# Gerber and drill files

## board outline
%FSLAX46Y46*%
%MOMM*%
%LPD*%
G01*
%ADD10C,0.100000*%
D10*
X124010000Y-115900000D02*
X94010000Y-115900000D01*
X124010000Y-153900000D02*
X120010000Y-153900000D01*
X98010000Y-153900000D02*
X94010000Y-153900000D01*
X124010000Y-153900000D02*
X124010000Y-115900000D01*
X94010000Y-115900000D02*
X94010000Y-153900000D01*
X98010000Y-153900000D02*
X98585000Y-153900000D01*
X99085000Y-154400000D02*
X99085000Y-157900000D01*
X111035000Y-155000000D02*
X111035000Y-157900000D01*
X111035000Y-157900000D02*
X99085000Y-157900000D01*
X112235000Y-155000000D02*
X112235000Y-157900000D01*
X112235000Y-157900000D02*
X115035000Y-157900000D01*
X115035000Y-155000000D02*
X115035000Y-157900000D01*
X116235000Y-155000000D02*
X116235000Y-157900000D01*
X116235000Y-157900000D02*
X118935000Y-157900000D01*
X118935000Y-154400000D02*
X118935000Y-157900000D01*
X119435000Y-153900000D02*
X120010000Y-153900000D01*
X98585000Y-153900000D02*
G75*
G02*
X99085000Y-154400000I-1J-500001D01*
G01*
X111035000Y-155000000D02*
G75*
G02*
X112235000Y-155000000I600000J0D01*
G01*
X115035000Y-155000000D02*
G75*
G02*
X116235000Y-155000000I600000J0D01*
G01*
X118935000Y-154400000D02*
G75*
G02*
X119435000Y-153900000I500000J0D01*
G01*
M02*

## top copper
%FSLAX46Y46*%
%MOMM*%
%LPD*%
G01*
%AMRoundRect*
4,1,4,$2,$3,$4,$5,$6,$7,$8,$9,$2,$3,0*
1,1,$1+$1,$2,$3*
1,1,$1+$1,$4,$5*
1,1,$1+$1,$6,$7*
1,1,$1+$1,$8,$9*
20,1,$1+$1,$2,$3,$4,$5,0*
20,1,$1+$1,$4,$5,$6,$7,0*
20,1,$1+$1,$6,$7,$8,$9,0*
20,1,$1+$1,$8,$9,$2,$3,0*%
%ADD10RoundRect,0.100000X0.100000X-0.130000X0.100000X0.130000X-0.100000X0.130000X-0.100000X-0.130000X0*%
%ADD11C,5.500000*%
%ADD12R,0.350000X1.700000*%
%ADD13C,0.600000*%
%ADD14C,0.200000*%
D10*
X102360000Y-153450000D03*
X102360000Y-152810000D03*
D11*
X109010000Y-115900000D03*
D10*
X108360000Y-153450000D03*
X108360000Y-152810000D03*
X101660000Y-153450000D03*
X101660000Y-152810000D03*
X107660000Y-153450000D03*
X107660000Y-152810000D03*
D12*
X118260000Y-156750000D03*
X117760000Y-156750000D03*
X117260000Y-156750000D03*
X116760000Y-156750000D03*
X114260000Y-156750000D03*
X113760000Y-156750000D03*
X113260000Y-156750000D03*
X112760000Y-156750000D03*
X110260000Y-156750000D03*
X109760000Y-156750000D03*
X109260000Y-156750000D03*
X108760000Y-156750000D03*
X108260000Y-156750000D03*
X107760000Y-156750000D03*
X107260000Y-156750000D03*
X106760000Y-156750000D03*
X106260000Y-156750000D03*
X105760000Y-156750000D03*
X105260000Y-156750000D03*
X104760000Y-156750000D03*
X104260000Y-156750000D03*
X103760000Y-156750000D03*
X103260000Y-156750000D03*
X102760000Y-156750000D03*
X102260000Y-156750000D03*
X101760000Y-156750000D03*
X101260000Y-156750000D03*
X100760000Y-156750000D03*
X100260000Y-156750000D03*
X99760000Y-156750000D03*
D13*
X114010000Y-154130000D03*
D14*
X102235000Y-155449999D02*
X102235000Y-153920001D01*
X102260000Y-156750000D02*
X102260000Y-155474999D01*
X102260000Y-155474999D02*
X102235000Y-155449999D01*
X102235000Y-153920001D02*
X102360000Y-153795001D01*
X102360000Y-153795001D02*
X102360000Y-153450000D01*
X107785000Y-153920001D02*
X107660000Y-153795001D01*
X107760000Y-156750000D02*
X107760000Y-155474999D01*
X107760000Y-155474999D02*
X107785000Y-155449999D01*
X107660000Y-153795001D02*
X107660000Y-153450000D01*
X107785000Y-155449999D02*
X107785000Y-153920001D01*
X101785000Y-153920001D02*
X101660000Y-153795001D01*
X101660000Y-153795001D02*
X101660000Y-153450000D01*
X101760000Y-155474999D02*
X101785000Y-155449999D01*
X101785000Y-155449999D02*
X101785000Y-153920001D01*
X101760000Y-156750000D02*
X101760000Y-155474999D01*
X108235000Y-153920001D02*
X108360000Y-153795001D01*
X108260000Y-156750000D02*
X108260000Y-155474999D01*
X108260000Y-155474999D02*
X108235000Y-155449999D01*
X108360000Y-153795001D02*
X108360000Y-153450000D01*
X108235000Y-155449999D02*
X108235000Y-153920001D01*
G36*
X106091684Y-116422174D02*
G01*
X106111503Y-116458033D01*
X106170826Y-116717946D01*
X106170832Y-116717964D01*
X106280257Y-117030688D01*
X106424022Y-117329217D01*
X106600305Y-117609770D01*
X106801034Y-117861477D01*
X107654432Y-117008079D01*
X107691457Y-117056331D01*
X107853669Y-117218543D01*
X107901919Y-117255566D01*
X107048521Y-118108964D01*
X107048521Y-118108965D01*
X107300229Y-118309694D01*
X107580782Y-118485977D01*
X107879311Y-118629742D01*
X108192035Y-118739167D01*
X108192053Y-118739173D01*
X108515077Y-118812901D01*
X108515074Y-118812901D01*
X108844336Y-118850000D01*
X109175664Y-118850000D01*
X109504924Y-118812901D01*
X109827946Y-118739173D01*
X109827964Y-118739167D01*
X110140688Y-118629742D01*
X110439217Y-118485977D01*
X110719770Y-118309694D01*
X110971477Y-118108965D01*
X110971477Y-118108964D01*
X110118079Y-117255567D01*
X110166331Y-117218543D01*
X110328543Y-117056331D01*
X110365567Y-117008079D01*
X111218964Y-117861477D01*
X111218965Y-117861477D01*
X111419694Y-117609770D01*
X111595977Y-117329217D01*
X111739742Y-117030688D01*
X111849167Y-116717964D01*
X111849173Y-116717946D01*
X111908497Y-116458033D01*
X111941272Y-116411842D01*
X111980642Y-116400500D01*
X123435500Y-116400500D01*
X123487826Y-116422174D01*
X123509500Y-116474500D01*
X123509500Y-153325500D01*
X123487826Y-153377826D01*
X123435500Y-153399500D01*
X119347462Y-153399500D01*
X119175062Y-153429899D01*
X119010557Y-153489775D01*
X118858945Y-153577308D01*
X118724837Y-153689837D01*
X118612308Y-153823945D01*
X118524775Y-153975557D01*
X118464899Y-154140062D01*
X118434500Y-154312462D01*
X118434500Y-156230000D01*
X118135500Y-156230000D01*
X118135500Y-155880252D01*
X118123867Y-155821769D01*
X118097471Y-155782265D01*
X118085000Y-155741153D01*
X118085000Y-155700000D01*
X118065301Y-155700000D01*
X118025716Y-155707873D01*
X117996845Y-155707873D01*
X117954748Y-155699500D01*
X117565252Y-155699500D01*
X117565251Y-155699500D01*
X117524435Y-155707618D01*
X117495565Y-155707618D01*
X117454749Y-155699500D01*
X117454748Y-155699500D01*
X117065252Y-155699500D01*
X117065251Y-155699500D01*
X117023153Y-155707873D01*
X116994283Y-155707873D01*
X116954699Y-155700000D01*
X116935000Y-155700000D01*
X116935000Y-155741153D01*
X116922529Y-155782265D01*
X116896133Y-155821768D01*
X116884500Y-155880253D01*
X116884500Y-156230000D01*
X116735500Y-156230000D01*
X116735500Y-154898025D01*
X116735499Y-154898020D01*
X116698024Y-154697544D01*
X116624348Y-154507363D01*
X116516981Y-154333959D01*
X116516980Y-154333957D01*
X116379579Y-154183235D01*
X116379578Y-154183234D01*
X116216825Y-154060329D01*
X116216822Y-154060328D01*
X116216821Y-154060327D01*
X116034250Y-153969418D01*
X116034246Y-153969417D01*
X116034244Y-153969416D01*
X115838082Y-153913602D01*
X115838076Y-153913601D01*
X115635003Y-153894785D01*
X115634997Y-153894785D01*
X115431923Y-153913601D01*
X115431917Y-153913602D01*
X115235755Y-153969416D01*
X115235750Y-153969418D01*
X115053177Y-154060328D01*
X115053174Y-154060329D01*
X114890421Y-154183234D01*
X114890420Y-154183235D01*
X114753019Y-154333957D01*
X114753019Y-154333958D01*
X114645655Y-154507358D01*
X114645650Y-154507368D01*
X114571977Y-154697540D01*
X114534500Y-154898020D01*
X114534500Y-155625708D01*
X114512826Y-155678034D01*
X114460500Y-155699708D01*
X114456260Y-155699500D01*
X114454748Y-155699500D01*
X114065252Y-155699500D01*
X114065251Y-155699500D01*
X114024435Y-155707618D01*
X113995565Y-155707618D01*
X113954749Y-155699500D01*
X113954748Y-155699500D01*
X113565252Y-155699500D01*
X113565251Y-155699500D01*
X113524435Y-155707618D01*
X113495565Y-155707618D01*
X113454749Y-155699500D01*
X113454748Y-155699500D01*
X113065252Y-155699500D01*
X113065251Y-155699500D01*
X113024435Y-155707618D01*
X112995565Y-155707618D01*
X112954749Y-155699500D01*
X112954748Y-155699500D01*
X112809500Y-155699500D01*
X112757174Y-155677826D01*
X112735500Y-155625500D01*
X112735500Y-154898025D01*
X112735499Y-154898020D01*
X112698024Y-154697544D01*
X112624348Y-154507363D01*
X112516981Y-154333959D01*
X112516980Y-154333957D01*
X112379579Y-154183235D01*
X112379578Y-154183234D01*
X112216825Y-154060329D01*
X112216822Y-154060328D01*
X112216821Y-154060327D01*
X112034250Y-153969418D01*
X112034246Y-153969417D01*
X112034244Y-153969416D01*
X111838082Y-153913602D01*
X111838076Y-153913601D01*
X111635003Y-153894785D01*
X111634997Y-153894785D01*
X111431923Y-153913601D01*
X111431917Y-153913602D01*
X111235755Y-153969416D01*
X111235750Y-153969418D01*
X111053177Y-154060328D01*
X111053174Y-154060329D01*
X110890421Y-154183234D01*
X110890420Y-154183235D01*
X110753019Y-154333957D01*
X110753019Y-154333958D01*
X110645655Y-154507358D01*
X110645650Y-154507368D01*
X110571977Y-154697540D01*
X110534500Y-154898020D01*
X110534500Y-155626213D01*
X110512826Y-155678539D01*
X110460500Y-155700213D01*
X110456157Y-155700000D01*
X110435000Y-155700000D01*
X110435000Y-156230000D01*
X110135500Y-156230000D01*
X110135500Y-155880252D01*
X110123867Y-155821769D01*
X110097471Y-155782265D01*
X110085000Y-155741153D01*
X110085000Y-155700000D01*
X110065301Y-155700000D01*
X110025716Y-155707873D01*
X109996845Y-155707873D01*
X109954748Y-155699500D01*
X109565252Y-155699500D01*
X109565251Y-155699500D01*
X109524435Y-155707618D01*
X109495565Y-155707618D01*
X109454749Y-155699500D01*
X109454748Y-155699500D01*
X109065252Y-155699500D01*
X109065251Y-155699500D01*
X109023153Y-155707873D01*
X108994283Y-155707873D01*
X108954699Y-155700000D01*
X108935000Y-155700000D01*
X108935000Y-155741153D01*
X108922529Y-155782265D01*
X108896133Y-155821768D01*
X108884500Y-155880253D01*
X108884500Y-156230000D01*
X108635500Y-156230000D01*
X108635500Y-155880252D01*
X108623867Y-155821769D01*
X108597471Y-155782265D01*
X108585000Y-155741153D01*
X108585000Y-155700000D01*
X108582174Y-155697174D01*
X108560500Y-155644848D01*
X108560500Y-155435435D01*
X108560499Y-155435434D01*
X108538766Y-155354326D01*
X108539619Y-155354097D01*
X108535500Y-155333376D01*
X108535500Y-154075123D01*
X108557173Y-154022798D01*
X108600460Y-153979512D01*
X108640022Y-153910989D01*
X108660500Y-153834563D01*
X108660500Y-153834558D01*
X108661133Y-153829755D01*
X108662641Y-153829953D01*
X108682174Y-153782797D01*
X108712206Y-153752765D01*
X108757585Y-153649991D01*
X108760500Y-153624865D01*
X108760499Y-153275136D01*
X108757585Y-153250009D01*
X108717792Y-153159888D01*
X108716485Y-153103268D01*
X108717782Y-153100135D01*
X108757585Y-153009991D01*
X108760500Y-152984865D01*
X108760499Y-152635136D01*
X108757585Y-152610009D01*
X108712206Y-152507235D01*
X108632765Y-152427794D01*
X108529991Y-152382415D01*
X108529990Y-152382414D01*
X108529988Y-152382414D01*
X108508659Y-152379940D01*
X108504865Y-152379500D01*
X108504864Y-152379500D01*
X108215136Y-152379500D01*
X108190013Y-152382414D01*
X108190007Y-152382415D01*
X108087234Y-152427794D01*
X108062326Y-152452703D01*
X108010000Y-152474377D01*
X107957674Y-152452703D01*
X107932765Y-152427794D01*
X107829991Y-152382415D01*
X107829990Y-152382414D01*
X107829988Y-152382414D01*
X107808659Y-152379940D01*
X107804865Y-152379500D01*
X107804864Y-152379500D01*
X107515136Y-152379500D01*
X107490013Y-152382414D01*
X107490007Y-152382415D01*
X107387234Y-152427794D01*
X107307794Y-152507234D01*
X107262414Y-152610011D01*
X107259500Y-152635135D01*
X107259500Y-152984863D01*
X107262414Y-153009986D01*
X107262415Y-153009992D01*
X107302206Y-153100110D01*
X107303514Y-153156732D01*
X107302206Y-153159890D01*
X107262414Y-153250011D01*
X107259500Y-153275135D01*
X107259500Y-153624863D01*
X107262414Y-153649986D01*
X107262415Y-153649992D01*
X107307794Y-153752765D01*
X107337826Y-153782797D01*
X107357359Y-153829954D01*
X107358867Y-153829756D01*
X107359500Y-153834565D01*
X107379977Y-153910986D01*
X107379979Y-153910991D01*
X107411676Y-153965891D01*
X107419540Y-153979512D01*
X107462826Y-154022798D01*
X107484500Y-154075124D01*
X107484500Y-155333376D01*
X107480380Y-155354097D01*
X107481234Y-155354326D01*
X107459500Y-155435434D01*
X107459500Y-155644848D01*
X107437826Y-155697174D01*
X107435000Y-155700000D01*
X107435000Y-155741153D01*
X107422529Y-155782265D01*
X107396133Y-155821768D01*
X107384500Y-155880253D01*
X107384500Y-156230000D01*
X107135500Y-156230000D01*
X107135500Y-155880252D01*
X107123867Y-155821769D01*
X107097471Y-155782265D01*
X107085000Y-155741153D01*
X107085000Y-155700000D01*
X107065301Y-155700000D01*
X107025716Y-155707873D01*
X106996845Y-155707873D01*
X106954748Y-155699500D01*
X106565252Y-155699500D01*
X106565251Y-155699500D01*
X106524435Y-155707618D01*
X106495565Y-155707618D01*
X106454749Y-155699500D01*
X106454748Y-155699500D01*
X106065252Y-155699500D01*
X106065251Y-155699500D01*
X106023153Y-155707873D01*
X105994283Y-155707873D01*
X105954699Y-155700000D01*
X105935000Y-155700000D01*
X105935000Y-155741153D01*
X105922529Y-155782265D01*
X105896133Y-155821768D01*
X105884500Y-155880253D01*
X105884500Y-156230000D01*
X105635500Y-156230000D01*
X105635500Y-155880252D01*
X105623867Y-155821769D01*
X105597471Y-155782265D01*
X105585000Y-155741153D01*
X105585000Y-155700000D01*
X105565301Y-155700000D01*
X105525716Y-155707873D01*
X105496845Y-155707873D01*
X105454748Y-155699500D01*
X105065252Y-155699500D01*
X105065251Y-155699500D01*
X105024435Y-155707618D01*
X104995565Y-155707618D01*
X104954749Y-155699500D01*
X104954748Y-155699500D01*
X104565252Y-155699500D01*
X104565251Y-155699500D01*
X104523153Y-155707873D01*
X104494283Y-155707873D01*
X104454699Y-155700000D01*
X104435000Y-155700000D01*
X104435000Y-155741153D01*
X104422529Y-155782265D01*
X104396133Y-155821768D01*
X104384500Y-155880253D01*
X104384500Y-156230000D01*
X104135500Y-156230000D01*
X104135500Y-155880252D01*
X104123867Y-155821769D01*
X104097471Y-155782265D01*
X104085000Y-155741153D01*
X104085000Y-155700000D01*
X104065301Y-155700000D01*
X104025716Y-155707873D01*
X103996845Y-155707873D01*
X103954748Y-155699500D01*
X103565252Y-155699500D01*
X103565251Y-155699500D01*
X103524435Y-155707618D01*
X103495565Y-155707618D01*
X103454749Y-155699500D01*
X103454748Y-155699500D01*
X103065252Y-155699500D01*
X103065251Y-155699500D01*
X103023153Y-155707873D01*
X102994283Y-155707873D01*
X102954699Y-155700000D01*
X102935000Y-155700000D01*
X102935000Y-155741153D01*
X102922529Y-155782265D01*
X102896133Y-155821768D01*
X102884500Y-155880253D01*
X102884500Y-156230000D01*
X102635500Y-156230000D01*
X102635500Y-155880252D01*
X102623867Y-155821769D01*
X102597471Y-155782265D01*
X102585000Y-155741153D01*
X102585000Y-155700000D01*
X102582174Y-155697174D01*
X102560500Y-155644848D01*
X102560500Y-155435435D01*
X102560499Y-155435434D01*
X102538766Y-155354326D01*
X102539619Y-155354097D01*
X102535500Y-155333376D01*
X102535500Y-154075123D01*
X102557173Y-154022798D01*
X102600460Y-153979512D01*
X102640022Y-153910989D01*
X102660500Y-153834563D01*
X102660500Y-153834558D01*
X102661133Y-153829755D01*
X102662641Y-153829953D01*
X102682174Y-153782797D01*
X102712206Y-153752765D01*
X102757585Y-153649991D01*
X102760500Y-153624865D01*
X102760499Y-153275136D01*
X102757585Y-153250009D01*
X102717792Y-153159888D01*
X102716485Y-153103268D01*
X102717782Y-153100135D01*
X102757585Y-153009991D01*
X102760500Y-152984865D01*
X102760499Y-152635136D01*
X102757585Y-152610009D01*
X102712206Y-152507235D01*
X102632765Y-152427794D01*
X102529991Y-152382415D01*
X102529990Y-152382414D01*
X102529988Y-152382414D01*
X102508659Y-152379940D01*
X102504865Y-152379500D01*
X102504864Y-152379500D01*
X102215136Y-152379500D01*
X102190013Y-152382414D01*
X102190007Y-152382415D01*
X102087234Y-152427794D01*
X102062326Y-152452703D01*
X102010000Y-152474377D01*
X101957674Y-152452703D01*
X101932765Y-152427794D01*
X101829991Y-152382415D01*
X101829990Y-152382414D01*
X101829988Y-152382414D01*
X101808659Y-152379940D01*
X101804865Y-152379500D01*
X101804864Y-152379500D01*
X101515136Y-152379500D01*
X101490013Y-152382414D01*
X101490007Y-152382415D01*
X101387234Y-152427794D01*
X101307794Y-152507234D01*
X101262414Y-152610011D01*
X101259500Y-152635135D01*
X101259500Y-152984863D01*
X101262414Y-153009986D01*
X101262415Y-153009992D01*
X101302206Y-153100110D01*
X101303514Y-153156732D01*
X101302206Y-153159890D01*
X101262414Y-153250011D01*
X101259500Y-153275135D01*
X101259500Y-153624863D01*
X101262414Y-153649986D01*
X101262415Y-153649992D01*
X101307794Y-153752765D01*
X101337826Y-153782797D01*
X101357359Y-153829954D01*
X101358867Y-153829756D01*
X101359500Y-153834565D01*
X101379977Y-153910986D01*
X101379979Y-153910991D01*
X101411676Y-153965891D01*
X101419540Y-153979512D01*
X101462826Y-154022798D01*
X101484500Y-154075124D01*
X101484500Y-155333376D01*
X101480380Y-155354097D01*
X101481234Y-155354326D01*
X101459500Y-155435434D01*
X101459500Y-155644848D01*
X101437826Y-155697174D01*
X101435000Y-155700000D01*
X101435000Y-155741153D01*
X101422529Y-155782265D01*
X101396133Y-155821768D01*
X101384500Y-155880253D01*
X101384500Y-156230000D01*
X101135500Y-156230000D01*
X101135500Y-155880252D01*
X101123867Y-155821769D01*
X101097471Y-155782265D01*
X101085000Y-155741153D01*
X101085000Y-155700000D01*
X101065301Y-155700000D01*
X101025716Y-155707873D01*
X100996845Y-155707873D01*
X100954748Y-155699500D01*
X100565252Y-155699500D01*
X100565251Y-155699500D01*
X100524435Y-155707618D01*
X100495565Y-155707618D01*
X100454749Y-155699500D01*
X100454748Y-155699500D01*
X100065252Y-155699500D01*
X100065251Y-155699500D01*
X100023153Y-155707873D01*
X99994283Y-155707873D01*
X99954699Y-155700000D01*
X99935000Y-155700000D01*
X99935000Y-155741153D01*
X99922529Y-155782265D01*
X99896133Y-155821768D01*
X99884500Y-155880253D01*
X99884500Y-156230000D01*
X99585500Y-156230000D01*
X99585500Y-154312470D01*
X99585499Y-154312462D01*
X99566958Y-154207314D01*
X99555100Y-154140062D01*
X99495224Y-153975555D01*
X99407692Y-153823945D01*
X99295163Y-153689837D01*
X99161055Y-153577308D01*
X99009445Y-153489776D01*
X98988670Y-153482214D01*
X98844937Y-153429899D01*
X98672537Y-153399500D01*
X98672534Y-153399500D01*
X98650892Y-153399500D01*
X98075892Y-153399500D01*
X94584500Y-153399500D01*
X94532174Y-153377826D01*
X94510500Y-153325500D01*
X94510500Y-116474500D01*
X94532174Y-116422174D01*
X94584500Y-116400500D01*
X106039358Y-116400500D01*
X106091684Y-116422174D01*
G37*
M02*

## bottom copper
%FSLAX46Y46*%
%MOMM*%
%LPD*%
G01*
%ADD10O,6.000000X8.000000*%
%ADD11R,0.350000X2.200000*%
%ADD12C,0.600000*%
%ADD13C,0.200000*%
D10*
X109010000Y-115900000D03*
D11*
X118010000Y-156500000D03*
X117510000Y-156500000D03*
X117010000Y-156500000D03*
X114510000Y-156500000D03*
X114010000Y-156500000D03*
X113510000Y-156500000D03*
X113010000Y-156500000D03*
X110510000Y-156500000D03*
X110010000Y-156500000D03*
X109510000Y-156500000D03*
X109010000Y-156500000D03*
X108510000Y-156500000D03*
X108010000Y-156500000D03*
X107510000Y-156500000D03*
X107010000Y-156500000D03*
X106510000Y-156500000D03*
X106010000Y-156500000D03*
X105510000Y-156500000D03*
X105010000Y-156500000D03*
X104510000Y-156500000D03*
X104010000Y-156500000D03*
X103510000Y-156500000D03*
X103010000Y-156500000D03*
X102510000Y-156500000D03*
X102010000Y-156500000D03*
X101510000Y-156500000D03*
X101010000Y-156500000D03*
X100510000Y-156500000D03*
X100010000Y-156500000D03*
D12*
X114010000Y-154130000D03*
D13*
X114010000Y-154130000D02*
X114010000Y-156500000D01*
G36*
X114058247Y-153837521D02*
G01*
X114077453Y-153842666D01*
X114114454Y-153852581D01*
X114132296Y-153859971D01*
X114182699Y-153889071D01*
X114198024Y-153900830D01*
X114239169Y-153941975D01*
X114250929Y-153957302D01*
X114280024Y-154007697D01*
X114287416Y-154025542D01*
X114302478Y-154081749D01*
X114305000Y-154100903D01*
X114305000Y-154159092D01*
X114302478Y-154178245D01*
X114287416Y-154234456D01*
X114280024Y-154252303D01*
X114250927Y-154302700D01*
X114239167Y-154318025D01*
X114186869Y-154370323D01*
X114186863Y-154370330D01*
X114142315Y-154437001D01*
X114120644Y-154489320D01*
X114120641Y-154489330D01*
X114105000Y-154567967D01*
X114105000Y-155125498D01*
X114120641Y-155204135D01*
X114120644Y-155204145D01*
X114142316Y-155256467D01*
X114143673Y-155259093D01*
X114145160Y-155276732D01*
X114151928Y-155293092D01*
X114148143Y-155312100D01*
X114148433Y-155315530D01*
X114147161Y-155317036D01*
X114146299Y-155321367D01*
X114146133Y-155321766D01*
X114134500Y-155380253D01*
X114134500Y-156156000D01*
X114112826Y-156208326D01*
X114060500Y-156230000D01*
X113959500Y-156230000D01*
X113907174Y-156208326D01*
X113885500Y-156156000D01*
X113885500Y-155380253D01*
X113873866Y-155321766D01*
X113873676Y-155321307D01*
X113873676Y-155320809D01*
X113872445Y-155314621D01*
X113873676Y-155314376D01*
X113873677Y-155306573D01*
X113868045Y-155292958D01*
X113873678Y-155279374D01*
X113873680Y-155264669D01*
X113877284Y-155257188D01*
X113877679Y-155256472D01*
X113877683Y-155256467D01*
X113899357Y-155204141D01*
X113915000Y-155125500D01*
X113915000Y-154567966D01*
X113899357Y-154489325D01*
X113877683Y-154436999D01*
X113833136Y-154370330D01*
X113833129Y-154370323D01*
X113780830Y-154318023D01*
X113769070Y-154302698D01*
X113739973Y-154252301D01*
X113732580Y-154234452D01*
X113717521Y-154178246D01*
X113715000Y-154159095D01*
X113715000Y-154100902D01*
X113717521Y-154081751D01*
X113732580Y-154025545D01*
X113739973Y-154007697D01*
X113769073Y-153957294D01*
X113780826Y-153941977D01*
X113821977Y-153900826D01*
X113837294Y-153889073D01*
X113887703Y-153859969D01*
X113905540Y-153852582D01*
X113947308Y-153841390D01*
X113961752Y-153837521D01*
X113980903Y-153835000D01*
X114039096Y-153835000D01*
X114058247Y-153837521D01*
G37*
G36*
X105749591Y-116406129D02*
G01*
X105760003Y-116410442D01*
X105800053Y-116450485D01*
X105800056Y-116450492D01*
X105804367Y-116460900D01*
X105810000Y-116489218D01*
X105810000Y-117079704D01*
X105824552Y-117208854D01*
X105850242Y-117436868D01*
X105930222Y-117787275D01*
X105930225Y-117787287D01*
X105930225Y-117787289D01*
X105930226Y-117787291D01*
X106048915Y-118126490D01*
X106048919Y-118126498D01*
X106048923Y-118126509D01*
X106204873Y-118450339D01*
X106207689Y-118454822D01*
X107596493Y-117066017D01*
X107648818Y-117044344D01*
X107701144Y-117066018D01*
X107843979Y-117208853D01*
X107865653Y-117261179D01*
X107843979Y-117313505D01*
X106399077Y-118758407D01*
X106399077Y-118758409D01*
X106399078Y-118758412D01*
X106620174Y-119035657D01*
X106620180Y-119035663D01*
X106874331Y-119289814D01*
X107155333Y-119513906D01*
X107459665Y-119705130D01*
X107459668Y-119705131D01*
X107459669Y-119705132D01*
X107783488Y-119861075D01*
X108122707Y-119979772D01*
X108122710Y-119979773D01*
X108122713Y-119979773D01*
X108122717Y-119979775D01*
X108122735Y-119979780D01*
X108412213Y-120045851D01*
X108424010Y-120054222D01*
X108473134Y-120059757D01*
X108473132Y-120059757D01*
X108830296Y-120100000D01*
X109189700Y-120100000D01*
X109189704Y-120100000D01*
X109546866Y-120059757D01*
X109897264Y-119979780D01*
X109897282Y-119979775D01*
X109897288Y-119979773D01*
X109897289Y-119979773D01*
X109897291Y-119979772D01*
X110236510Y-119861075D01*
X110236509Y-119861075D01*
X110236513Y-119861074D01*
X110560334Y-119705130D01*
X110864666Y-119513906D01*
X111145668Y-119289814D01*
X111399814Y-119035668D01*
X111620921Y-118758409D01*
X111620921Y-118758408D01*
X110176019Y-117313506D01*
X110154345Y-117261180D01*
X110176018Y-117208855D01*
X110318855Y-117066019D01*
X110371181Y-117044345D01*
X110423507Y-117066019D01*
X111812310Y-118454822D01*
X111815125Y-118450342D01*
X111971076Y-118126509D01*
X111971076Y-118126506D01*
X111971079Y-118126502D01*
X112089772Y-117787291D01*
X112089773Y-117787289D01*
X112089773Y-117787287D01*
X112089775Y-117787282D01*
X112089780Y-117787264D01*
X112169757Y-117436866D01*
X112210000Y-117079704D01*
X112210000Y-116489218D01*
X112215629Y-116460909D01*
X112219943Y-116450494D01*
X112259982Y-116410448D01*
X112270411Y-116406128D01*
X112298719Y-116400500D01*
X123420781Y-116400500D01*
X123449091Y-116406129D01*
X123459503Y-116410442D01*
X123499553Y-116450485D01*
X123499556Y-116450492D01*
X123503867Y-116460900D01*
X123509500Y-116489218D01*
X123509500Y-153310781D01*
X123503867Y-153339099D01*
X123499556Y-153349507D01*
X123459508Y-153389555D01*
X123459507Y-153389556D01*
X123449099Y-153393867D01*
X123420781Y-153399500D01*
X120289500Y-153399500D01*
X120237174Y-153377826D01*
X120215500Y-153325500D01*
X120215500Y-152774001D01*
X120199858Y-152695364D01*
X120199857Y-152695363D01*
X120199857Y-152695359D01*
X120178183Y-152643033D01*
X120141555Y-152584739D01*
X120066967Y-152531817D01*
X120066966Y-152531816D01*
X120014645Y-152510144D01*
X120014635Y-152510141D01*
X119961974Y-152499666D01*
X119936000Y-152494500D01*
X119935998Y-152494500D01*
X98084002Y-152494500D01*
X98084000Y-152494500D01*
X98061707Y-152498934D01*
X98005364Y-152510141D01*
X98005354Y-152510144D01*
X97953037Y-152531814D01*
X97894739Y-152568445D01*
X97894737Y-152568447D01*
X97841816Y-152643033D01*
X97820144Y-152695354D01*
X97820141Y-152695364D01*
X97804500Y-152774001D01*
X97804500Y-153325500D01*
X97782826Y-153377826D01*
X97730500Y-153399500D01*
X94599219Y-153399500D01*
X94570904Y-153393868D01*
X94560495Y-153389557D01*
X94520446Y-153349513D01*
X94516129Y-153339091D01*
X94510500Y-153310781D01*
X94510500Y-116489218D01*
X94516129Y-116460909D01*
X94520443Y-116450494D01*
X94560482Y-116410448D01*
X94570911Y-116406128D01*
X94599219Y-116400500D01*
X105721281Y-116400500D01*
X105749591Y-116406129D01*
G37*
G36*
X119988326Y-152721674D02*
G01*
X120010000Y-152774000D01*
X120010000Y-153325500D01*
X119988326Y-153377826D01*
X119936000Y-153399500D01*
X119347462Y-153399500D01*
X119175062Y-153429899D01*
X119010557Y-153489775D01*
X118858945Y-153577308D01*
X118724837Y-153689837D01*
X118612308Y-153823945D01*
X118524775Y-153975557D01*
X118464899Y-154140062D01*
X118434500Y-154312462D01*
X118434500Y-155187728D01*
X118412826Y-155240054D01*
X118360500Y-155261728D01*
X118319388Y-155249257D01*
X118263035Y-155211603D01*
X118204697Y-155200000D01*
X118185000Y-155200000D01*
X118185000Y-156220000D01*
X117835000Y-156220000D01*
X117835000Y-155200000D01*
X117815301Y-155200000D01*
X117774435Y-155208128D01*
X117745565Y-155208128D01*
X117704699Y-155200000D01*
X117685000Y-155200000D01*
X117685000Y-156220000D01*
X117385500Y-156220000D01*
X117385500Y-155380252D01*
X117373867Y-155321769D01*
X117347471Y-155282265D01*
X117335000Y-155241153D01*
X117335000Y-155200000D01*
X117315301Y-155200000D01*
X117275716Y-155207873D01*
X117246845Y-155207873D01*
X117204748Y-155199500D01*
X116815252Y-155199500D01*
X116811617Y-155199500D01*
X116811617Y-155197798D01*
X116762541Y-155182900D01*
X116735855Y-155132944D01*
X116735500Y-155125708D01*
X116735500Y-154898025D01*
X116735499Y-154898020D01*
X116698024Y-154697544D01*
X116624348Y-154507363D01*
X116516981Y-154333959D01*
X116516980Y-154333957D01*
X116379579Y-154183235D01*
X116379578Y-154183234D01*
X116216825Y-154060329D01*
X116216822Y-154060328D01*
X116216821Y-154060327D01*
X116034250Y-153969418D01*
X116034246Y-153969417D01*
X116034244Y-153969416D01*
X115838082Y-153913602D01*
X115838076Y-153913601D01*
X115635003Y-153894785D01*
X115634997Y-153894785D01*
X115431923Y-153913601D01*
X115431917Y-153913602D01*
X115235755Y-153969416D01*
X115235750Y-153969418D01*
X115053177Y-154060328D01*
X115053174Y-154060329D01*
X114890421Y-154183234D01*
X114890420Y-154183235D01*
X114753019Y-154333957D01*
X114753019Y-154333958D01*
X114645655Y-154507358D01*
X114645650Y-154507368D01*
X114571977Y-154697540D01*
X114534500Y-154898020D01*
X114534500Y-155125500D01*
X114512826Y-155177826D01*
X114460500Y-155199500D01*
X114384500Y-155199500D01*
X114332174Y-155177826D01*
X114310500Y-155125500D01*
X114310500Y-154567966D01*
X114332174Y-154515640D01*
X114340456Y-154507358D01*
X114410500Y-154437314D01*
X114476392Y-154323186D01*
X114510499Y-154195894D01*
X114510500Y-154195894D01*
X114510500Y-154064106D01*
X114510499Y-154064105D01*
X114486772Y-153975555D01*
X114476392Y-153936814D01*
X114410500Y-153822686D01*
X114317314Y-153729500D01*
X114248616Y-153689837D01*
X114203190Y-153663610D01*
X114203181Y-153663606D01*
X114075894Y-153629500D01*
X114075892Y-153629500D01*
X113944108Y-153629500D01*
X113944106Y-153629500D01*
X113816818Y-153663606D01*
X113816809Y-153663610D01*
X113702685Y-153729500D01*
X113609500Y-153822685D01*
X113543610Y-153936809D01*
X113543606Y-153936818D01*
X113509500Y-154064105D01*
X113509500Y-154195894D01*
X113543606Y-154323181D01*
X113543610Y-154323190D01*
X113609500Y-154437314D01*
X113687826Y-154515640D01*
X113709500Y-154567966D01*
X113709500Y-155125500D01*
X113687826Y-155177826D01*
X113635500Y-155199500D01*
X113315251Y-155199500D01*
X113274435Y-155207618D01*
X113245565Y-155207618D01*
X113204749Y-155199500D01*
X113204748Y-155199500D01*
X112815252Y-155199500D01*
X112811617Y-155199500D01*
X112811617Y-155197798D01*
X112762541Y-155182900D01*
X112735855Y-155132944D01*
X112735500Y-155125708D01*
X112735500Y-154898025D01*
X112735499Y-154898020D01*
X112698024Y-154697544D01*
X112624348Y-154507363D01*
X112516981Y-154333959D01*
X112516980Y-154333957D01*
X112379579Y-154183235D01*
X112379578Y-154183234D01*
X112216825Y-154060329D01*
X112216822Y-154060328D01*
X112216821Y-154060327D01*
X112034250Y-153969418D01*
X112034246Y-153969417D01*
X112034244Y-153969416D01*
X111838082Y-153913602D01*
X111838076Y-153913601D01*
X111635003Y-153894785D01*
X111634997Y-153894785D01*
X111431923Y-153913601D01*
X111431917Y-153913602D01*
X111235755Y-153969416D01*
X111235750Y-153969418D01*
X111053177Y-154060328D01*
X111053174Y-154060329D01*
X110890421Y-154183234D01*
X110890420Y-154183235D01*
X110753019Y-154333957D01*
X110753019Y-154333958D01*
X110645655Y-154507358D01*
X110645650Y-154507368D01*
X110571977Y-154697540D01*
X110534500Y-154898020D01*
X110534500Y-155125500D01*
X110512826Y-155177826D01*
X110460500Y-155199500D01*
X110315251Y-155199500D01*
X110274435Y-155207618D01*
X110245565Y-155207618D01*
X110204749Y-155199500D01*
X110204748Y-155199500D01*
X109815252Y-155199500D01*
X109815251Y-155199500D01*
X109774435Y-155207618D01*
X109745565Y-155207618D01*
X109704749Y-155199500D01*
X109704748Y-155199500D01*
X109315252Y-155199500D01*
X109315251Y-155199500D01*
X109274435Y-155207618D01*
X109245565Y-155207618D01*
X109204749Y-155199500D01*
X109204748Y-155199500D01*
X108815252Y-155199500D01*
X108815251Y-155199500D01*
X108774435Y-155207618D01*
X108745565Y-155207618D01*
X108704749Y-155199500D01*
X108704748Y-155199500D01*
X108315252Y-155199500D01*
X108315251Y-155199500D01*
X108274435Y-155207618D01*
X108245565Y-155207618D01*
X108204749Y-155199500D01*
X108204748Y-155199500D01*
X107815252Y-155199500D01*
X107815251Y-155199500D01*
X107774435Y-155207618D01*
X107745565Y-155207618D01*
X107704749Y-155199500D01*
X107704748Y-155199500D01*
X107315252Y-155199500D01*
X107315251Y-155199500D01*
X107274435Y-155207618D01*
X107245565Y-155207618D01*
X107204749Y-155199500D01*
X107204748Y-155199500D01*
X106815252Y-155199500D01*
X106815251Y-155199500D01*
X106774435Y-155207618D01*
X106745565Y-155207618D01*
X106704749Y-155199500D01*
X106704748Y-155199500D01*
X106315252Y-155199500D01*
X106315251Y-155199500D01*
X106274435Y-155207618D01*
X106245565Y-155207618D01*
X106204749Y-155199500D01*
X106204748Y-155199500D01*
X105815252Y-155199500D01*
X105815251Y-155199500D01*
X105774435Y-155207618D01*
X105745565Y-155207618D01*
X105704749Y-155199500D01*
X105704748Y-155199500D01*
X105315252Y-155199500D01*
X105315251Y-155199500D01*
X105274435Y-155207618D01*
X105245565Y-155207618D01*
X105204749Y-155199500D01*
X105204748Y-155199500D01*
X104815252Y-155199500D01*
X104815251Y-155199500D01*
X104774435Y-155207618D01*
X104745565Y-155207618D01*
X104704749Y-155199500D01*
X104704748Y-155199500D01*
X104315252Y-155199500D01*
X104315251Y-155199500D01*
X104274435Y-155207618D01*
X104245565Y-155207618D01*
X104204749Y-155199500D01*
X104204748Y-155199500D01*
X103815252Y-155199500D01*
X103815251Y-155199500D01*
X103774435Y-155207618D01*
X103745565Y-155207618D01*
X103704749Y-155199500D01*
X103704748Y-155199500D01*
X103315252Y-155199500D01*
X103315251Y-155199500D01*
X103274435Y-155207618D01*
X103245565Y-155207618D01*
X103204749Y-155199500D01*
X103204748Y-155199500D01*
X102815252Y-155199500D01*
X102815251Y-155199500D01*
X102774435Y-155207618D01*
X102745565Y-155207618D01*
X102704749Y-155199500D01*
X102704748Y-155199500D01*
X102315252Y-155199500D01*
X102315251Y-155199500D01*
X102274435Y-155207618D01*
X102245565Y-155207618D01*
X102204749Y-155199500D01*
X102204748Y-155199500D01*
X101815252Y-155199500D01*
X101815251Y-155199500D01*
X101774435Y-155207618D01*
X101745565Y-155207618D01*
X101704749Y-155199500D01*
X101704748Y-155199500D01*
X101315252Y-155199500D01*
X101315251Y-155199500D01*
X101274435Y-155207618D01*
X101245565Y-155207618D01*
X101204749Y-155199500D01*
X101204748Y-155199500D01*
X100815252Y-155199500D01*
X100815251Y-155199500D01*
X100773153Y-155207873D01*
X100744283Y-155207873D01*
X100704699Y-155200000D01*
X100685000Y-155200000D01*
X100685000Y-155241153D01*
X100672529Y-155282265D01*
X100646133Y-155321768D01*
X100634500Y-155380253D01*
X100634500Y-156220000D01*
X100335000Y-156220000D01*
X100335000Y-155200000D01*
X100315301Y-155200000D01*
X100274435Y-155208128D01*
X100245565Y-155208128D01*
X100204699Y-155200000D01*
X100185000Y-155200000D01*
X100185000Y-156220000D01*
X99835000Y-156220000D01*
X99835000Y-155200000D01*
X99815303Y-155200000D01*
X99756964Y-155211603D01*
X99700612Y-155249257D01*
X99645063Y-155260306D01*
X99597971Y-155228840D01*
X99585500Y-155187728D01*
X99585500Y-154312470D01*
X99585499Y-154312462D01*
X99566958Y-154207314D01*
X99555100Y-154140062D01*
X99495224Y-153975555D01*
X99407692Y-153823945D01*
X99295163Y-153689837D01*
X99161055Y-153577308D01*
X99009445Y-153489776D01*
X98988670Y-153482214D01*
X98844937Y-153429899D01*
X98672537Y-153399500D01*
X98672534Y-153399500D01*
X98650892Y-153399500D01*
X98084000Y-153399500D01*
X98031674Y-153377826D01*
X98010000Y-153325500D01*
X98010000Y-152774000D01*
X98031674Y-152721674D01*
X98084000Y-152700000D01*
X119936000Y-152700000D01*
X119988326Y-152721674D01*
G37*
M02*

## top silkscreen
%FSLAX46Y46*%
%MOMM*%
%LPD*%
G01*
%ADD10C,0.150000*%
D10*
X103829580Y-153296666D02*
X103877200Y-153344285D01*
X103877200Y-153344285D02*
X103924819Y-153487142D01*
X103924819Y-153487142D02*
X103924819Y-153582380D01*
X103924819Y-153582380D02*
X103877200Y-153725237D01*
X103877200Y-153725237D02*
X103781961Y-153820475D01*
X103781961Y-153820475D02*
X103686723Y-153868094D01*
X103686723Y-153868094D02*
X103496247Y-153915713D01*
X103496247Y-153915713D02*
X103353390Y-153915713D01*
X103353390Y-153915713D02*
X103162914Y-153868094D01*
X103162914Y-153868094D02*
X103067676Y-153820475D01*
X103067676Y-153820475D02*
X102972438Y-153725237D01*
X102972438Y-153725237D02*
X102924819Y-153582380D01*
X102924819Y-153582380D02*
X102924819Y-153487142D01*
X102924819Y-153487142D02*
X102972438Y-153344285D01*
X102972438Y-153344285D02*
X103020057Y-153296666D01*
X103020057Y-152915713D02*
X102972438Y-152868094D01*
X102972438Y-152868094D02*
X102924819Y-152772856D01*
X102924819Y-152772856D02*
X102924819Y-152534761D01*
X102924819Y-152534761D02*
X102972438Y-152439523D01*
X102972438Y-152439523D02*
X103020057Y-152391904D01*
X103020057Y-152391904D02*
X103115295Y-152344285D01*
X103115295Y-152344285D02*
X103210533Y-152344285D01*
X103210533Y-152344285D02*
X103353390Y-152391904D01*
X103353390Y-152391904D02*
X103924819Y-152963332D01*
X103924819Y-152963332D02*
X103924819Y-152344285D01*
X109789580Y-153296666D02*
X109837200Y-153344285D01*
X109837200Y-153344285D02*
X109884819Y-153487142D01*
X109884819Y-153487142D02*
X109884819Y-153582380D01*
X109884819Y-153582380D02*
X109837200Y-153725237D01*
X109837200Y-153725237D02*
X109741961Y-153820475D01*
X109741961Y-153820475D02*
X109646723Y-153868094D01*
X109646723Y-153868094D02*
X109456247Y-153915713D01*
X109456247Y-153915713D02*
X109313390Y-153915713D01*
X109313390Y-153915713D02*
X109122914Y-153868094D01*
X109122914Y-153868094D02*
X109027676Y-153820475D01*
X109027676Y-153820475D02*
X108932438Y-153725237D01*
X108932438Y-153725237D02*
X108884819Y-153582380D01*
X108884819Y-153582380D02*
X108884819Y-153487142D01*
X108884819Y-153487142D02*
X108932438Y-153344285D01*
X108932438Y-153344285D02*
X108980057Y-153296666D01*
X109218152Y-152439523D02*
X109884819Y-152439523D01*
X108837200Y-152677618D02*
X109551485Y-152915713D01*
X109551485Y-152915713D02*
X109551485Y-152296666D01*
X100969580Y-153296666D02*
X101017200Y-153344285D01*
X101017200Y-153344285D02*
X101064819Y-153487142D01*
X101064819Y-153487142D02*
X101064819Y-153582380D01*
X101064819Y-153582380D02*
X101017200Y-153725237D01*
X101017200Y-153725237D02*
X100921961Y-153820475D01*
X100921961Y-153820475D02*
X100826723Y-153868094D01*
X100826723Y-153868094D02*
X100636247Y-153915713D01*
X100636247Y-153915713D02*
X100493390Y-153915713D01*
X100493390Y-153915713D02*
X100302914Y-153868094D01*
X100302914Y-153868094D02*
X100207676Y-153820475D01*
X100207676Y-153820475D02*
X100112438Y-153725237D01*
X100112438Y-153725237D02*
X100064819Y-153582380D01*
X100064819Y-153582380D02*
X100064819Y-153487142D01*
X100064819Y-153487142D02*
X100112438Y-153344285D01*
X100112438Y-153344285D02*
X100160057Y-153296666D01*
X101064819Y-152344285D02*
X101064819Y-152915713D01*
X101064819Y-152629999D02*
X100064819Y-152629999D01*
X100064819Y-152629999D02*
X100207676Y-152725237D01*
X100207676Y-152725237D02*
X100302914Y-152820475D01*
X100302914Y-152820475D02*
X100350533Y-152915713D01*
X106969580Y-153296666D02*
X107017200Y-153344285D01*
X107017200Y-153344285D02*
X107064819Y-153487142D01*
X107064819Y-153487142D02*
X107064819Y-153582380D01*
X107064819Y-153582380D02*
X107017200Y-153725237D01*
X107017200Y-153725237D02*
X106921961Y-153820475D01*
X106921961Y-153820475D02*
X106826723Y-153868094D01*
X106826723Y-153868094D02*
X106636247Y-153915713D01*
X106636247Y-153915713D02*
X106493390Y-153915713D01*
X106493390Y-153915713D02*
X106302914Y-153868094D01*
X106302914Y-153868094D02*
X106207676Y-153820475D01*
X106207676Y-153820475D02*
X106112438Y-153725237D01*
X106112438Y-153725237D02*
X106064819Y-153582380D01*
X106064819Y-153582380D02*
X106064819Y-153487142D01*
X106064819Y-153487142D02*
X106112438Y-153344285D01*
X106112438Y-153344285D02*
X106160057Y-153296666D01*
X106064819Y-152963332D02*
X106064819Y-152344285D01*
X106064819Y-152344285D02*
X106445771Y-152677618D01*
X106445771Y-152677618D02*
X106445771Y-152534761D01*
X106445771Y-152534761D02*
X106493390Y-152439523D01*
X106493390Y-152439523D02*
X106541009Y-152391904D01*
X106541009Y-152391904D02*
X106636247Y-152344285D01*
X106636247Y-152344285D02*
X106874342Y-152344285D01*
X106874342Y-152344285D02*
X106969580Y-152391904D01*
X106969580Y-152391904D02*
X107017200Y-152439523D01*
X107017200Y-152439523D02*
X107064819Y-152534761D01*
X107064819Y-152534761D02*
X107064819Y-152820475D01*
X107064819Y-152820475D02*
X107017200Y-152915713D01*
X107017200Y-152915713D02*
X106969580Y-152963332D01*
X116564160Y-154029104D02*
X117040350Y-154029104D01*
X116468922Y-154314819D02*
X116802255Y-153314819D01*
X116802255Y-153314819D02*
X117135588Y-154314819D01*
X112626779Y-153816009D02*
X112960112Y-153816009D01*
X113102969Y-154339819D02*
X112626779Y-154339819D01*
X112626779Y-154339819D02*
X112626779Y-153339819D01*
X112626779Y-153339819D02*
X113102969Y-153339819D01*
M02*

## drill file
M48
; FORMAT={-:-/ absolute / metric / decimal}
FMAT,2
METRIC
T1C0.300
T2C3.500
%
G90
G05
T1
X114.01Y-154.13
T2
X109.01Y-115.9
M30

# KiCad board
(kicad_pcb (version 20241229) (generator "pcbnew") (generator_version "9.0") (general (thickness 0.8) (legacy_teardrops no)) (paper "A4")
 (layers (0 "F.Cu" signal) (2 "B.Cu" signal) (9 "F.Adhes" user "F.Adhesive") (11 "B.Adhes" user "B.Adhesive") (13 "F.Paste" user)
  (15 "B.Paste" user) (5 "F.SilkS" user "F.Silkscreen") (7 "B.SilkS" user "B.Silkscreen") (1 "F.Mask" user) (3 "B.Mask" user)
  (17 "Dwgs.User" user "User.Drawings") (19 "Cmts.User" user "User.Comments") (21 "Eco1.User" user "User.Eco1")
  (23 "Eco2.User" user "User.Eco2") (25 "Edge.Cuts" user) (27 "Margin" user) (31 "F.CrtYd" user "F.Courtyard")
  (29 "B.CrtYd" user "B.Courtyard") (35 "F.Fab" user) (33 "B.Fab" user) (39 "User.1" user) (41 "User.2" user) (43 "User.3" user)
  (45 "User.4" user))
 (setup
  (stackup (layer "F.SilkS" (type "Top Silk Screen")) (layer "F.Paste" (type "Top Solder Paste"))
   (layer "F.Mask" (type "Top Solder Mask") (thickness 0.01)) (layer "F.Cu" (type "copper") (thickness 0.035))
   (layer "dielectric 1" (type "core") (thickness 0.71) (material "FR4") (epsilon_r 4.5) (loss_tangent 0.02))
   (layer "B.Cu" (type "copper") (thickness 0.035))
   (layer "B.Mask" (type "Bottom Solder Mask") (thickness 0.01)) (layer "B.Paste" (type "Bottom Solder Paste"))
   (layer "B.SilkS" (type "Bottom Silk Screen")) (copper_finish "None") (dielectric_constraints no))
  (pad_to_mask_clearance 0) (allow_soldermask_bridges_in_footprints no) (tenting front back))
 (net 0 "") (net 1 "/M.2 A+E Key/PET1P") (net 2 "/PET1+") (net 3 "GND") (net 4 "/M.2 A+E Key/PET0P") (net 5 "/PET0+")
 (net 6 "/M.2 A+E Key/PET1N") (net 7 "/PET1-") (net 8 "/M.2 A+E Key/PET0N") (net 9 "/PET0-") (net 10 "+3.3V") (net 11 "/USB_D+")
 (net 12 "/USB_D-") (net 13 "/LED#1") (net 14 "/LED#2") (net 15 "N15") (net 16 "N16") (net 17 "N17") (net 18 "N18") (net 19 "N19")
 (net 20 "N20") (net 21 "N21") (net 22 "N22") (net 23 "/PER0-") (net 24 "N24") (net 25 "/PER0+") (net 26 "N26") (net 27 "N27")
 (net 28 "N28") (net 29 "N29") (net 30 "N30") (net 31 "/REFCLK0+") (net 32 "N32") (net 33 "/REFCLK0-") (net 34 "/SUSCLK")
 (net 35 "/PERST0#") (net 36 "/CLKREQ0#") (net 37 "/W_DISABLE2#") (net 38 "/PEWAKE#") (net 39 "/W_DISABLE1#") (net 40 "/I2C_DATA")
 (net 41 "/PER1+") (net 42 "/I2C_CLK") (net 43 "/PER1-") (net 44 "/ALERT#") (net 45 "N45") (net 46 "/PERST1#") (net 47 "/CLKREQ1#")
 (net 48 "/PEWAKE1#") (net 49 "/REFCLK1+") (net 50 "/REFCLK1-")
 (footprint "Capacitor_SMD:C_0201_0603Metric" (layer "F.Cu") (at 102.36 153.13 90)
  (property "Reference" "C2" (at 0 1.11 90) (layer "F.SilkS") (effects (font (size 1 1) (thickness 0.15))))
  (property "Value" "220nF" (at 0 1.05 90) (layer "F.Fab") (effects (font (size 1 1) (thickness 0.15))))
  (pad "" smd roundrect (at -0.345 0 90) (size 0.318 0.36) (layers "F.Paste") (roundrect_rratio 0.25))
  (pad "" smd roundrect (at 0.345 0 90) (size 0.318 0.36) (layers "F.Paste") (roundrect_rratio 0.25))
  (pad "1" smd roundrect (at -0.32 0 90) (size 0.46 0.4) (layers "F.Cu" "F.Mask") (roundrect_rratio 0.25) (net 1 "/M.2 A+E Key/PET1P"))
  (pad "2" smd roundrect (at 0.32 0 90) (size 0.46 0.4) (layers "F.Cu" "F.Mask") (roundrect_rratio 0.25) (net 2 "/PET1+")))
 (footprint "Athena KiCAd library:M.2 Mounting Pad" (layer "F.Cu") (at 109.01 115.9)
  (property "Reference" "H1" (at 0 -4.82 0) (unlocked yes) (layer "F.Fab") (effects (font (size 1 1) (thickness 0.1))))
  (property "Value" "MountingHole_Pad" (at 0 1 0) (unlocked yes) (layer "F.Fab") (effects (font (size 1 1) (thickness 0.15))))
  (pad "1" thru_hole circle (at 0 0) (size 5.5 5.5) (drill 3.5) (layers "*.Cu" "*.Mask") (remove_unused_layers no) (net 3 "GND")
   (padstack (mode front_inner_back)
    (layer "Inner" (shape circle) (size 5.5 5.5) (zone_connect -1))
    (layer "B.Cu" (shape oval) (size 6 8) (thermal_bridge_angle 45) (zone_connect -1)))))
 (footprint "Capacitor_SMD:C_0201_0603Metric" (layer "F.Cu") (at 108.36 153.13 90)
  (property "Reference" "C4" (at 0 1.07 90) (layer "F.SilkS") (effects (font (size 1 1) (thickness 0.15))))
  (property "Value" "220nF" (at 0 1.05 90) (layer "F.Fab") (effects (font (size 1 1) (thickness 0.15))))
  (pad "" smd roundrect (at -0.345 0 90) (size 0.318 0.36) (layers "F.Paste") (roundrect_rratio 0.25))
  (pad "" smd roundrect (at 0.345 0 90) (size 0.318 0.36) (layers "F.Paste") (roundrect_rratio 0.25))
  (pad "1" smd roundrect (at -0.32 0 90) (size 0.46 0.4) (layers "F.Cu" "F.Mask") (roundrect_rratio 0.25) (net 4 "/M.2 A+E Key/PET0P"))
  (pad "2" smd roundrect (at 0.32 0 90) (size 0.46 0.4) (layers "F.Cu" "F.Mask") (roundrect_rratio 0.25) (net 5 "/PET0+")))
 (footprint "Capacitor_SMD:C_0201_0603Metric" (layer "F.Cu") (at 101.66 153.13 90)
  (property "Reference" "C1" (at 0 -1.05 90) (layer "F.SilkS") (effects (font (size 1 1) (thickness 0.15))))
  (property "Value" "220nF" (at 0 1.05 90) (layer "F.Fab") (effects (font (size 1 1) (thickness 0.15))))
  (pad "" smd roundrect (at -0.345 0 90) (size 0.318 0.36) (layers "F.Paste") (roundrect_rratio 0.25))
  (pad "" smd roundrect (at 0.345 0 90) (size 0.318 0.36) (layers "F.Paste") (roundrect_rratio 0.25))
  (pad "1" smd roundrect (at -0.32 0 90) (size 0.46 0.4) (layers "F.Cu" "F.Mask") (roundrect_rratio 0.25) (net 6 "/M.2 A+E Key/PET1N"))
  (pad "2" smd roundrect (at 0.32 0 90) (size 0.46 0.4) (layers "F.Cu" "F.Mask") (roundrect_rratio 0.25) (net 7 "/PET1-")))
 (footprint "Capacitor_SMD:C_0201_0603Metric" (layer "F.Cu") (at 107.66 153.13 90)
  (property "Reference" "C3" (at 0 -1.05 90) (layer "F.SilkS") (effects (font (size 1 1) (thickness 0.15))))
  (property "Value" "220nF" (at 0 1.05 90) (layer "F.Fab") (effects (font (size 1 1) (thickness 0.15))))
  (pad "" smd roundrect (at -0.345 0 90) (size 0.318 0.36) (layers "F.Paste") (roundrect_rratio 0.25))
  (pad "" smd roundrect (at 0.345 0 90) (size 0.318 0.36) (layers "F.Paste") (roundrect_rratio 0.25))
  (pad "1" smd roundrect (at -0.32 0 90) (size 0.46 0.4) (layers "F.Cu" "F.Mask") (roundrect_rratio 0.25) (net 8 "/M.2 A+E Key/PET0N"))
  (pad "2" smd roundrect (at 0.32 0 90) (size 0.46 0.4) (layers "F.Cu" "F.Mask") (roundrect_rratio 0.25) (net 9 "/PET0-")))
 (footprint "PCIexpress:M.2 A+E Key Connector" (layer "F.Cu") (at 109.01 156.79)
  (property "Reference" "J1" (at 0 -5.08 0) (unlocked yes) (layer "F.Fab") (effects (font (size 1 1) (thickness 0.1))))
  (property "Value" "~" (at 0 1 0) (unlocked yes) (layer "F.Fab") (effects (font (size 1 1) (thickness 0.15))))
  (fp_line (start -11 -2.89) (end -10.425 -2.89) (stroke (width 0.1) (type default)) (layer "Edge.Cuts") (net 3))
  (fp_line (start -9.925 -2.39) (end -9.925 1.11) (stroke (width 0.1) (type default)) (layer "Edge.Cuts") (net 3))
  (fp_line (start 2.025 -1.79) (end 2.025 1.11) (stroke (width 0.1) (type default)) (layer "Edge.Cuts") (net 3))
  (fp_line (start 2.025 1.11) (end -9.925 1.11) (stroke (width 0.1) (type default)) (layer "Edge.Cuts") (net 3))
  (fp_line (start 3.225 -1.79) (end 3.225 1.11) (stroke (width 0.1) (type default)) (layer "Edge.Cuts") (net 3))
  (fp_line (start 3.225 1.11) (end 6.025 1.11) (stroke (width 0.1) (type default)) (layer "Edge.Cuts") (net 3))
  (fp_line (start 6.025 -1.79) (end 6.025 1.11) (stroke (width 0.1) (type default)) (layer "Edge.Cuts") (net 3))
  (fp_line (start 7.225 -1.79) (end 7.225 1.11) (stroke (width 0.1) (type default)) (layer "Edge.Cuts") (net 3))
  (fp_line (start 7.225 1.11) (end 9.925 1.11) (stroke (width 0.1) (type default)) (layer "Edge.Cuts") (net 3))
  (fp_line (start 9.925 -2.39) (end 9.925 1.11) (stroke (width 0.1) (type default)) (layer "Edge.Cuts") (net 3))
  (fp_line (start 10.425 -2.89) (end 11 -2.89) (stroke (width 0.1) (type default)) (layer "Edge.Cuts") (net 3))
  (fp_arc (start -10.425 -2.89) (mid -10.071447 -2.743553) (end -9.925 -2.39) (stroke (width 0.1) (type default)) (layer "Edge.Cuts")
   (net 3))
  (fp_arc (start 2.025 -1.79) (mid 2.625 -2.39) (end 3.225 -1.79) (stroke (width 0.1) (type default)) (layer "Edge.Cuts") (net 3))
  (fp_arc (start 6.025 -1.79) (mid 6.625 -2.39) (end 7.225 -1.79) (stroke (width 0.1) (type default)) (layer "Edge.Cuts") (net 3))
  (fp_arc (start 9.925 -2.39) (mid 10.071447 -2.743553) (end 10.425 -2.89) (stroke (width 0.1) (type default)) (layer "Edge.Cuts") (net 3))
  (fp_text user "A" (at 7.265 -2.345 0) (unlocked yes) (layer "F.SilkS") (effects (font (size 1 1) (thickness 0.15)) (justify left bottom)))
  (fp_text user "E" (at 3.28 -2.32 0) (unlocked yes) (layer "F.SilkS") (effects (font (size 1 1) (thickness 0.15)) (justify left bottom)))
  (pad "1" smd rect (at 9.25 -0.04 180) (size 0.35 1.7) (layers "F.Cu") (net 3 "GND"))
  (pad "2" smd rect (at 9 -0.29 180) (size 0.35 2.2) (layers "B.Cu") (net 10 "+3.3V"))
  (pad "3" smd rect (at 8.75 -0.04 180) (size 0.35 1.7) (layers "F.Cu") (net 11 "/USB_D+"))
  (pad "4" smd rect (at 8.5 -0.29 180) (size 0.35 2.2) (layers "B.Cu") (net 10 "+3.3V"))
  (pad "5" smd rect (at 8.25 -0.04 180) (size 0.35 1.7) (layers "F.Cu") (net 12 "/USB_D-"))
  (pad "6" smd rect (at 8 -0.29 180) (size 0.35 2.2) (layers "B.Cu") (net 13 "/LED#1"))
  (pad "7" smd rect (at 7.75 -0.04 180) (size 0.35 1.7) (layers "F.Cu") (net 3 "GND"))
  (pad "16" smd rect (at 5.5 -0.29 180) (size 0.35 2.2) (layers "B.Cu") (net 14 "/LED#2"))
  (pad "17" smd rect (at 5.25 -0.04 180) (size 0.35 1.7) (layers "F.Cu") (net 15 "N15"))
  (pad "18" smd rect (at 5 -0.29 180) (size 0.35 2.2) (layers "B.Cu") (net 3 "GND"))
  (pad "19" smd rect (at 4.75 -0.04 180) (size 0.35 1.7) (layers "F.Cu") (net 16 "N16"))
  (pad "20" smd rect (at 4.5 -0.29 180) (size 0.35 2.2) (layers "B.Cu") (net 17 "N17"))
  (pad "21" smd rect (at 4.25 -0.04 180) (size 0.35 1.7) (layers "F.Cu") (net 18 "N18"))
  (pad "22" smd rect (at 4 -0.29 180) (size 0.35 2.2) (layers "B.Cu") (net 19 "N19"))
  (pad "23" smd rect (at 3.75 -0.04 180) (size 0.35 1.7) (layers "F.Cu") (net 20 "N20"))
  (pad "32" smd rect (at 1.5 -0.29 180) (size 0.35 2.2) (layers "B.Cu") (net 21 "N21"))
  (pad "33" smd rect (at 1.25 -0.04 180) (size 0.35 1.7) (layers "F.Cu") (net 3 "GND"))
  (pad "34" smd rect (at 1 -0.29 180) (size 0.35 2.2) (layers "B.Cu") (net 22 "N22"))
  (pad "35" smd rect (at 0.75 -0.04 180) (size 0.35 1.7) (layers "F.Cu") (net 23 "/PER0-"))
  (pad "36" smd rect (at 0.5 -0.29 180) (size 0.35 2.2) (layers "B.Cu") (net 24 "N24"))
  (pad "37" smd rect (at 0.25 -0.04 180) (size 0.35 1.7) (layers "F.Cu") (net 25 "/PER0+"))
  (pad "38" smd rect (at 0 -0.29 180) (size 0.35 2.2) (layers "B.Cu") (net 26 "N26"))
  (pad "39" smd rect (at -0.25 -0.04 180) (size 0.35 1.7) (layers "F.Cu") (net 3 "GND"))
  (pad "40" smd rect (at -0.5 -0.29 180) (size 0.35 2.2) (layers "B.Cu") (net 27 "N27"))
  (pad "41" smd rect (at -0.75 -0.04 180) (size 0.35 1.7) (layers "F.Cu") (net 4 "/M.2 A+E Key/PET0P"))
  (pad "42" smd rect (at -1 -0.29 180) (size 0.35 2.2) (layers "B.Cu") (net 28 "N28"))
  (pad "43" smd rect (at -1.25 -0.04 180) (size 0.35 1.7) (layers "F.Cu") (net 8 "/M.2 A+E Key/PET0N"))
  (pad "44" smd rect (at -1.5 -0.29 180) (size 0.35 2.2) (layers "B.Cu") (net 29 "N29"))
  (pad "45" smd rect (at -1.75 -0.04 180) (size 0.35 1.7) (layers "F.Cu") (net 3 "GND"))
  (pad "46" smd rect (at -2 -0.29 180) (size 0.35 2.2) (layers "B.Cu") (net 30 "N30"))
  (pad "47" smd rect (at -2.25 -0.04 180) (size 0.35 1.7) (layers "F.Cu") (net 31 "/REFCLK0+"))
  (pad "48" smd rect (at -2.5 -0.29 180) (size 0.35 2.2) (layers "B.Cu") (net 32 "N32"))
  (pad "49" smd rect (at -2.75 -0.04 180) (size 0.35 1.7) (layers "F.Cu") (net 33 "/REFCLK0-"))
  (pad "50" smd rect (at -3 -0.29 180) (size 0.35 2.2) (layers "B.Cu") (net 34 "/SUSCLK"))
  (pad "51" smd rect (at -3.25 -0.04 180) (size 0.35 1.7) (layers "F.Cu") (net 3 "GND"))
  (pad "52" smd rect (at -3.5 -0.29 180) (size 0.35 2.2) (layers "B.Cu") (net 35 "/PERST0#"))
  (pad "53" smd rect (at -3.75 -0.04 180) (size 0.35 1.7) (layers "F.Cu") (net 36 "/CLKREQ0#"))
  (pad "54" smd rect (at -4 -0.29 180) (size 0.35 2.2) (layers "B.Cu") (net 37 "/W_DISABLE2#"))
  (pad "55" smd rect (at -4.25 -0.04 180) (size 0.35 1.7) (layers "F.Cu") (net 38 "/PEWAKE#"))
  (pad "56" smd rect (at -4.5 -0.29 180) (size 0.35 2.2) (layers "B.Cu") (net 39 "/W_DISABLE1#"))
  (pad "57" smd rect (at -4.75 -0.04 180) (size 0.35 1.7) (layers "F.Cu") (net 3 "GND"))
  (pad "58" smd rect (at -5 -0.29 180) (size 0.35 2.2) (layers "B.Cu") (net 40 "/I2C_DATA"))
  (pad "59" smd rect (at -5.25 -0.04 180) (size 0.35 1.7) (layers "F.Cu") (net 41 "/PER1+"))
  (pad "60" smd rect (at -5.5 -0.29 180) (size 0.35 2.2) (layers "B.Cu") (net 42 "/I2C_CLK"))
  (pad "61" smd rect (at -5.75 -0.04 180) (size 0.35 1.7) (layers "F.Cu") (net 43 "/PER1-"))
  (pad "62" smd rect (at -6 -0.29 180) (size 0.35 2.2) (layers "B.Cu") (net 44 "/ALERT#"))
  (pad "63" smd rect (at -6.25 -0.04 180) (size 0.35 1.7) (layers "F.Cu") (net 3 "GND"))
  (pad "64" smd rect (at -6.5 -0.29 180) (size 0.35 2.2) (layers "B.Cu") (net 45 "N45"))
  (pad "65" smd rect (at -6.75 -0.04 180) (size 0.35 1.7) (layers "F.Cu") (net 1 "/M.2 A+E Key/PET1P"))
  (pad "66" smd rect (at -7 -0.29 180) (size 0.35 2.2) (layers "B.Cu") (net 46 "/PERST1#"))
  (pad "67" smd rect (at -7.25 -0.04 180) (size 0.35 1.7) (layers "F.Cu") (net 6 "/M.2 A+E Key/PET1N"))
  (pad "68" smd rect (at -7.5 -0.29 180) (size 0.35 2.2) (layers "B.Cu") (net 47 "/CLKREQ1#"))
  (pad "69" smd rect (at -7.75 -0.04 180) (size 0.35 1.7) (layers "F.Cu") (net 3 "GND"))
  (pad "70" smd rect (at -8 -0.29 180) (size 0.35 2.2) (layers "B.Cu") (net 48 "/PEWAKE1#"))
  (pad "71" smd rect (at -8.25 -0.04 180) (size 0.35 1.7) (layers "F.Cu") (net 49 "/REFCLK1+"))
  (pad "72" smd rect (at -8.5 -0.29 180) (size 0.35 2.2) (layers "B.Cu") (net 10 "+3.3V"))
  (pad "73" smd rect (at -8.75 -0.04 180) (size 0.35 1.7) (layers "F.Cu") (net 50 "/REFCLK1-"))
  (pad "74" smd rect (at -9 -0.29 180) (size 0.35 2.2) (layers "B.Cu") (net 10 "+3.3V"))
  (pad "75" smd rect (at -9.25 -0.04 180) (size 0.35 1.7) (layers "F.Cu") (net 3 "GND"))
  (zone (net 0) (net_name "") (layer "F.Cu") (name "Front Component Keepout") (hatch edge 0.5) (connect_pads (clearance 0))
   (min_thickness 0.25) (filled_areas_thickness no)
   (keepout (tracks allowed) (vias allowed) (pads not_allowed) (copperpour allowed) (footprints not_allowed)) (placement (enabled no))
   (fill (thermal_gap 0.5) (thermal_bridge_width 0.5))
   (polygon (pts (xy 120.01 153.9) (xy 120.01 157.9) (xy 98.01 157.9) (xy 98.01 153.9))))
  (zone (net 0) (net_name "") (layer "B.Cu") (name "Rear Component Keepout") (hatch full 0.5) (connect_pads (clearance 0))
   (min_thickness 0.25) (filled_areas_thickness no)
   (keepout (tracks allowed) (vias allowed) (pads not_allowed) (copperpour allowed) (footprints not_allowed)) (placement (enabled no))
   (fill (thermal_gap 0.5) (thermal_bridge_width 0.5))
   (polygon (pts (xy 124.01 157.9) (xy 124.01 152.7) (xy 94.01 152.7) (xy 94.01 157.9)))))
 (gr_line (start 124.01 115.9) (end 94.01 115.9) (stroke (width 0.1) (type default)) (layer "Edge.Cuts"))
 (gr_line (start 124.01 153.9) (end 120.01 153.9) (stroke (width 0.1) (type default)) (layer "Edge.Cuts"))
 (gr_line (start 98.01 153.9) (end 94.01 153.9) (stroke (width 0.1) (type default)) (layer "Edge.Cuts"))
 (gr_line (start 124.01 153.9) (end 124.01 115.9) (stroke (width 0.1) (type default)) (layer "Edge.Cuts"))
 (gr_line (start 94.01 115.9) (end 94.01 153.9) (stroke (width 0.1) (type default)) (layer "Edge.Cuts"))
 (via (at 114.01 154.13) (size 0.6) (drill 0.3) (layers "F.Cu" "B.Cu") (free yes) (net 3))
 (segment (start 114.01 154.13) (end 114.01 156.5) (width 0.2) (layer "B.Cu") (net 3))
 (segment (start 102.235 155.449999) (end 102.235 153.920001) (width 0.2) (layer "F.Cu") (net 1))
 (segment (start 102.26 156.75) (end 102.26 155.474999) (width 0.2) (layer "F.Cu") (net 1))
 (segment (start 102.26 155.474999) (end 102.235 155.449999) (width 0.2) (layer "F.Cu") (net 1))
 (segment (start 102.235 153.920001) (end 102.36 153.795001) (width 0.2) (layer "F.Cu") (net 1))
 (segment (start 102.36 153.795001) (end 102.36 153.45) (width 0.2) (layer "F.Cu") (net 1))
 (segment (start 107.785 153.920001) (end 107.66 153.795001) (width 0.2) (layer "F.Cu") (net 8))
 (segment (start 107.76 156.75) (end 107.76 155.474999) (width 0.2) (layer "F.Cu") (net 8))
 (segment (start 107.76 155.474999) (end 107.785 155.449999) (width 0.2) (layer "F.Cu") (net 8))
 (segment (start 107.66 153.795001) (end 107.66 153.45) (width 0.2) (layer "F.Cu") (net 8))
 (segment (start 107.785 155.449999) (end 107.785 153.920001) (width 0.2) (layer "F.Cu") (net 8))
 (segment (start 101.785 153.920001) (end 101.66 153.795001) (width 0.2) (layer "F.Cu") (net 6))
 (segment (start 101.66 153.795001) (end 101.66 153.45) (width 0.2) (layer "F.Cu") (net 6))
 (segment (start 101.76 155.474999) (end 101.785 155.449999) (width 0.2) (layer "F.Cu") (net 6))
 (segment (start 101.785 155.449999) (end 101.785 153.920001) (width 0.2) (layer "F.Cu") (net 6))
 (segment (start 101.76 156.75) (end 101.76 155.474999) (width 0.2) (layer "F.Cu") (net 6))
 (segment (start 108.235 153.920001) (end 108.36 153.795001) (width 0.2) (layer "F.Cu") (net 4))
 (segment (start 108.26 156.75) (end 108.26 155.474999) (width 0.2) (layer "F.Cu") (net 4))
 (segment (start 108.26 155.474999) (end 108.235 155.449999) (width 0.2) (layer "F.Cu") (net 4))
 (segment (start 108.36 153.795001) (end 108.36 153.45) (width 0.2) (layer "F.Cu") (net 4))
 (segment (start 108.235 155.449999) (end 108.235 153.920001) (width 0.2) (layer "F.Cu") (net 4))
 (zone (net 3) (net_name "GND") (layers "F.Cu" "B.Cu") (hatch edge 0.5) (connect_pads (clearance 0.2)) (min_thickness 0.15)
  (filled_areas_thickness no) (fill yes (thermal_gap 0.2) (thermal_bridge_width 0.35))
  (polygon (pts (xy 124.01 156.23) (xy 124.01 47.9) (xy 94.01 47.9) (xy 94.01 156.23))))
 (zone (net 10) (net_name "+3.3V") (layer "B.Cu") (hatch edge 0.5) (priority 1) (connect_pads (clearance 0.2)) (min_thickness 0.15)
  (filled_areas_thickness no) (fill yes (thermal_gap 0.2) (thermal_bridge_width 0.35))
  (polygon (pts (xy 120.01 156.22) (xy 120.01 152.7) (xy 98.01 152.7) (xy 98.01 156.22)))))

